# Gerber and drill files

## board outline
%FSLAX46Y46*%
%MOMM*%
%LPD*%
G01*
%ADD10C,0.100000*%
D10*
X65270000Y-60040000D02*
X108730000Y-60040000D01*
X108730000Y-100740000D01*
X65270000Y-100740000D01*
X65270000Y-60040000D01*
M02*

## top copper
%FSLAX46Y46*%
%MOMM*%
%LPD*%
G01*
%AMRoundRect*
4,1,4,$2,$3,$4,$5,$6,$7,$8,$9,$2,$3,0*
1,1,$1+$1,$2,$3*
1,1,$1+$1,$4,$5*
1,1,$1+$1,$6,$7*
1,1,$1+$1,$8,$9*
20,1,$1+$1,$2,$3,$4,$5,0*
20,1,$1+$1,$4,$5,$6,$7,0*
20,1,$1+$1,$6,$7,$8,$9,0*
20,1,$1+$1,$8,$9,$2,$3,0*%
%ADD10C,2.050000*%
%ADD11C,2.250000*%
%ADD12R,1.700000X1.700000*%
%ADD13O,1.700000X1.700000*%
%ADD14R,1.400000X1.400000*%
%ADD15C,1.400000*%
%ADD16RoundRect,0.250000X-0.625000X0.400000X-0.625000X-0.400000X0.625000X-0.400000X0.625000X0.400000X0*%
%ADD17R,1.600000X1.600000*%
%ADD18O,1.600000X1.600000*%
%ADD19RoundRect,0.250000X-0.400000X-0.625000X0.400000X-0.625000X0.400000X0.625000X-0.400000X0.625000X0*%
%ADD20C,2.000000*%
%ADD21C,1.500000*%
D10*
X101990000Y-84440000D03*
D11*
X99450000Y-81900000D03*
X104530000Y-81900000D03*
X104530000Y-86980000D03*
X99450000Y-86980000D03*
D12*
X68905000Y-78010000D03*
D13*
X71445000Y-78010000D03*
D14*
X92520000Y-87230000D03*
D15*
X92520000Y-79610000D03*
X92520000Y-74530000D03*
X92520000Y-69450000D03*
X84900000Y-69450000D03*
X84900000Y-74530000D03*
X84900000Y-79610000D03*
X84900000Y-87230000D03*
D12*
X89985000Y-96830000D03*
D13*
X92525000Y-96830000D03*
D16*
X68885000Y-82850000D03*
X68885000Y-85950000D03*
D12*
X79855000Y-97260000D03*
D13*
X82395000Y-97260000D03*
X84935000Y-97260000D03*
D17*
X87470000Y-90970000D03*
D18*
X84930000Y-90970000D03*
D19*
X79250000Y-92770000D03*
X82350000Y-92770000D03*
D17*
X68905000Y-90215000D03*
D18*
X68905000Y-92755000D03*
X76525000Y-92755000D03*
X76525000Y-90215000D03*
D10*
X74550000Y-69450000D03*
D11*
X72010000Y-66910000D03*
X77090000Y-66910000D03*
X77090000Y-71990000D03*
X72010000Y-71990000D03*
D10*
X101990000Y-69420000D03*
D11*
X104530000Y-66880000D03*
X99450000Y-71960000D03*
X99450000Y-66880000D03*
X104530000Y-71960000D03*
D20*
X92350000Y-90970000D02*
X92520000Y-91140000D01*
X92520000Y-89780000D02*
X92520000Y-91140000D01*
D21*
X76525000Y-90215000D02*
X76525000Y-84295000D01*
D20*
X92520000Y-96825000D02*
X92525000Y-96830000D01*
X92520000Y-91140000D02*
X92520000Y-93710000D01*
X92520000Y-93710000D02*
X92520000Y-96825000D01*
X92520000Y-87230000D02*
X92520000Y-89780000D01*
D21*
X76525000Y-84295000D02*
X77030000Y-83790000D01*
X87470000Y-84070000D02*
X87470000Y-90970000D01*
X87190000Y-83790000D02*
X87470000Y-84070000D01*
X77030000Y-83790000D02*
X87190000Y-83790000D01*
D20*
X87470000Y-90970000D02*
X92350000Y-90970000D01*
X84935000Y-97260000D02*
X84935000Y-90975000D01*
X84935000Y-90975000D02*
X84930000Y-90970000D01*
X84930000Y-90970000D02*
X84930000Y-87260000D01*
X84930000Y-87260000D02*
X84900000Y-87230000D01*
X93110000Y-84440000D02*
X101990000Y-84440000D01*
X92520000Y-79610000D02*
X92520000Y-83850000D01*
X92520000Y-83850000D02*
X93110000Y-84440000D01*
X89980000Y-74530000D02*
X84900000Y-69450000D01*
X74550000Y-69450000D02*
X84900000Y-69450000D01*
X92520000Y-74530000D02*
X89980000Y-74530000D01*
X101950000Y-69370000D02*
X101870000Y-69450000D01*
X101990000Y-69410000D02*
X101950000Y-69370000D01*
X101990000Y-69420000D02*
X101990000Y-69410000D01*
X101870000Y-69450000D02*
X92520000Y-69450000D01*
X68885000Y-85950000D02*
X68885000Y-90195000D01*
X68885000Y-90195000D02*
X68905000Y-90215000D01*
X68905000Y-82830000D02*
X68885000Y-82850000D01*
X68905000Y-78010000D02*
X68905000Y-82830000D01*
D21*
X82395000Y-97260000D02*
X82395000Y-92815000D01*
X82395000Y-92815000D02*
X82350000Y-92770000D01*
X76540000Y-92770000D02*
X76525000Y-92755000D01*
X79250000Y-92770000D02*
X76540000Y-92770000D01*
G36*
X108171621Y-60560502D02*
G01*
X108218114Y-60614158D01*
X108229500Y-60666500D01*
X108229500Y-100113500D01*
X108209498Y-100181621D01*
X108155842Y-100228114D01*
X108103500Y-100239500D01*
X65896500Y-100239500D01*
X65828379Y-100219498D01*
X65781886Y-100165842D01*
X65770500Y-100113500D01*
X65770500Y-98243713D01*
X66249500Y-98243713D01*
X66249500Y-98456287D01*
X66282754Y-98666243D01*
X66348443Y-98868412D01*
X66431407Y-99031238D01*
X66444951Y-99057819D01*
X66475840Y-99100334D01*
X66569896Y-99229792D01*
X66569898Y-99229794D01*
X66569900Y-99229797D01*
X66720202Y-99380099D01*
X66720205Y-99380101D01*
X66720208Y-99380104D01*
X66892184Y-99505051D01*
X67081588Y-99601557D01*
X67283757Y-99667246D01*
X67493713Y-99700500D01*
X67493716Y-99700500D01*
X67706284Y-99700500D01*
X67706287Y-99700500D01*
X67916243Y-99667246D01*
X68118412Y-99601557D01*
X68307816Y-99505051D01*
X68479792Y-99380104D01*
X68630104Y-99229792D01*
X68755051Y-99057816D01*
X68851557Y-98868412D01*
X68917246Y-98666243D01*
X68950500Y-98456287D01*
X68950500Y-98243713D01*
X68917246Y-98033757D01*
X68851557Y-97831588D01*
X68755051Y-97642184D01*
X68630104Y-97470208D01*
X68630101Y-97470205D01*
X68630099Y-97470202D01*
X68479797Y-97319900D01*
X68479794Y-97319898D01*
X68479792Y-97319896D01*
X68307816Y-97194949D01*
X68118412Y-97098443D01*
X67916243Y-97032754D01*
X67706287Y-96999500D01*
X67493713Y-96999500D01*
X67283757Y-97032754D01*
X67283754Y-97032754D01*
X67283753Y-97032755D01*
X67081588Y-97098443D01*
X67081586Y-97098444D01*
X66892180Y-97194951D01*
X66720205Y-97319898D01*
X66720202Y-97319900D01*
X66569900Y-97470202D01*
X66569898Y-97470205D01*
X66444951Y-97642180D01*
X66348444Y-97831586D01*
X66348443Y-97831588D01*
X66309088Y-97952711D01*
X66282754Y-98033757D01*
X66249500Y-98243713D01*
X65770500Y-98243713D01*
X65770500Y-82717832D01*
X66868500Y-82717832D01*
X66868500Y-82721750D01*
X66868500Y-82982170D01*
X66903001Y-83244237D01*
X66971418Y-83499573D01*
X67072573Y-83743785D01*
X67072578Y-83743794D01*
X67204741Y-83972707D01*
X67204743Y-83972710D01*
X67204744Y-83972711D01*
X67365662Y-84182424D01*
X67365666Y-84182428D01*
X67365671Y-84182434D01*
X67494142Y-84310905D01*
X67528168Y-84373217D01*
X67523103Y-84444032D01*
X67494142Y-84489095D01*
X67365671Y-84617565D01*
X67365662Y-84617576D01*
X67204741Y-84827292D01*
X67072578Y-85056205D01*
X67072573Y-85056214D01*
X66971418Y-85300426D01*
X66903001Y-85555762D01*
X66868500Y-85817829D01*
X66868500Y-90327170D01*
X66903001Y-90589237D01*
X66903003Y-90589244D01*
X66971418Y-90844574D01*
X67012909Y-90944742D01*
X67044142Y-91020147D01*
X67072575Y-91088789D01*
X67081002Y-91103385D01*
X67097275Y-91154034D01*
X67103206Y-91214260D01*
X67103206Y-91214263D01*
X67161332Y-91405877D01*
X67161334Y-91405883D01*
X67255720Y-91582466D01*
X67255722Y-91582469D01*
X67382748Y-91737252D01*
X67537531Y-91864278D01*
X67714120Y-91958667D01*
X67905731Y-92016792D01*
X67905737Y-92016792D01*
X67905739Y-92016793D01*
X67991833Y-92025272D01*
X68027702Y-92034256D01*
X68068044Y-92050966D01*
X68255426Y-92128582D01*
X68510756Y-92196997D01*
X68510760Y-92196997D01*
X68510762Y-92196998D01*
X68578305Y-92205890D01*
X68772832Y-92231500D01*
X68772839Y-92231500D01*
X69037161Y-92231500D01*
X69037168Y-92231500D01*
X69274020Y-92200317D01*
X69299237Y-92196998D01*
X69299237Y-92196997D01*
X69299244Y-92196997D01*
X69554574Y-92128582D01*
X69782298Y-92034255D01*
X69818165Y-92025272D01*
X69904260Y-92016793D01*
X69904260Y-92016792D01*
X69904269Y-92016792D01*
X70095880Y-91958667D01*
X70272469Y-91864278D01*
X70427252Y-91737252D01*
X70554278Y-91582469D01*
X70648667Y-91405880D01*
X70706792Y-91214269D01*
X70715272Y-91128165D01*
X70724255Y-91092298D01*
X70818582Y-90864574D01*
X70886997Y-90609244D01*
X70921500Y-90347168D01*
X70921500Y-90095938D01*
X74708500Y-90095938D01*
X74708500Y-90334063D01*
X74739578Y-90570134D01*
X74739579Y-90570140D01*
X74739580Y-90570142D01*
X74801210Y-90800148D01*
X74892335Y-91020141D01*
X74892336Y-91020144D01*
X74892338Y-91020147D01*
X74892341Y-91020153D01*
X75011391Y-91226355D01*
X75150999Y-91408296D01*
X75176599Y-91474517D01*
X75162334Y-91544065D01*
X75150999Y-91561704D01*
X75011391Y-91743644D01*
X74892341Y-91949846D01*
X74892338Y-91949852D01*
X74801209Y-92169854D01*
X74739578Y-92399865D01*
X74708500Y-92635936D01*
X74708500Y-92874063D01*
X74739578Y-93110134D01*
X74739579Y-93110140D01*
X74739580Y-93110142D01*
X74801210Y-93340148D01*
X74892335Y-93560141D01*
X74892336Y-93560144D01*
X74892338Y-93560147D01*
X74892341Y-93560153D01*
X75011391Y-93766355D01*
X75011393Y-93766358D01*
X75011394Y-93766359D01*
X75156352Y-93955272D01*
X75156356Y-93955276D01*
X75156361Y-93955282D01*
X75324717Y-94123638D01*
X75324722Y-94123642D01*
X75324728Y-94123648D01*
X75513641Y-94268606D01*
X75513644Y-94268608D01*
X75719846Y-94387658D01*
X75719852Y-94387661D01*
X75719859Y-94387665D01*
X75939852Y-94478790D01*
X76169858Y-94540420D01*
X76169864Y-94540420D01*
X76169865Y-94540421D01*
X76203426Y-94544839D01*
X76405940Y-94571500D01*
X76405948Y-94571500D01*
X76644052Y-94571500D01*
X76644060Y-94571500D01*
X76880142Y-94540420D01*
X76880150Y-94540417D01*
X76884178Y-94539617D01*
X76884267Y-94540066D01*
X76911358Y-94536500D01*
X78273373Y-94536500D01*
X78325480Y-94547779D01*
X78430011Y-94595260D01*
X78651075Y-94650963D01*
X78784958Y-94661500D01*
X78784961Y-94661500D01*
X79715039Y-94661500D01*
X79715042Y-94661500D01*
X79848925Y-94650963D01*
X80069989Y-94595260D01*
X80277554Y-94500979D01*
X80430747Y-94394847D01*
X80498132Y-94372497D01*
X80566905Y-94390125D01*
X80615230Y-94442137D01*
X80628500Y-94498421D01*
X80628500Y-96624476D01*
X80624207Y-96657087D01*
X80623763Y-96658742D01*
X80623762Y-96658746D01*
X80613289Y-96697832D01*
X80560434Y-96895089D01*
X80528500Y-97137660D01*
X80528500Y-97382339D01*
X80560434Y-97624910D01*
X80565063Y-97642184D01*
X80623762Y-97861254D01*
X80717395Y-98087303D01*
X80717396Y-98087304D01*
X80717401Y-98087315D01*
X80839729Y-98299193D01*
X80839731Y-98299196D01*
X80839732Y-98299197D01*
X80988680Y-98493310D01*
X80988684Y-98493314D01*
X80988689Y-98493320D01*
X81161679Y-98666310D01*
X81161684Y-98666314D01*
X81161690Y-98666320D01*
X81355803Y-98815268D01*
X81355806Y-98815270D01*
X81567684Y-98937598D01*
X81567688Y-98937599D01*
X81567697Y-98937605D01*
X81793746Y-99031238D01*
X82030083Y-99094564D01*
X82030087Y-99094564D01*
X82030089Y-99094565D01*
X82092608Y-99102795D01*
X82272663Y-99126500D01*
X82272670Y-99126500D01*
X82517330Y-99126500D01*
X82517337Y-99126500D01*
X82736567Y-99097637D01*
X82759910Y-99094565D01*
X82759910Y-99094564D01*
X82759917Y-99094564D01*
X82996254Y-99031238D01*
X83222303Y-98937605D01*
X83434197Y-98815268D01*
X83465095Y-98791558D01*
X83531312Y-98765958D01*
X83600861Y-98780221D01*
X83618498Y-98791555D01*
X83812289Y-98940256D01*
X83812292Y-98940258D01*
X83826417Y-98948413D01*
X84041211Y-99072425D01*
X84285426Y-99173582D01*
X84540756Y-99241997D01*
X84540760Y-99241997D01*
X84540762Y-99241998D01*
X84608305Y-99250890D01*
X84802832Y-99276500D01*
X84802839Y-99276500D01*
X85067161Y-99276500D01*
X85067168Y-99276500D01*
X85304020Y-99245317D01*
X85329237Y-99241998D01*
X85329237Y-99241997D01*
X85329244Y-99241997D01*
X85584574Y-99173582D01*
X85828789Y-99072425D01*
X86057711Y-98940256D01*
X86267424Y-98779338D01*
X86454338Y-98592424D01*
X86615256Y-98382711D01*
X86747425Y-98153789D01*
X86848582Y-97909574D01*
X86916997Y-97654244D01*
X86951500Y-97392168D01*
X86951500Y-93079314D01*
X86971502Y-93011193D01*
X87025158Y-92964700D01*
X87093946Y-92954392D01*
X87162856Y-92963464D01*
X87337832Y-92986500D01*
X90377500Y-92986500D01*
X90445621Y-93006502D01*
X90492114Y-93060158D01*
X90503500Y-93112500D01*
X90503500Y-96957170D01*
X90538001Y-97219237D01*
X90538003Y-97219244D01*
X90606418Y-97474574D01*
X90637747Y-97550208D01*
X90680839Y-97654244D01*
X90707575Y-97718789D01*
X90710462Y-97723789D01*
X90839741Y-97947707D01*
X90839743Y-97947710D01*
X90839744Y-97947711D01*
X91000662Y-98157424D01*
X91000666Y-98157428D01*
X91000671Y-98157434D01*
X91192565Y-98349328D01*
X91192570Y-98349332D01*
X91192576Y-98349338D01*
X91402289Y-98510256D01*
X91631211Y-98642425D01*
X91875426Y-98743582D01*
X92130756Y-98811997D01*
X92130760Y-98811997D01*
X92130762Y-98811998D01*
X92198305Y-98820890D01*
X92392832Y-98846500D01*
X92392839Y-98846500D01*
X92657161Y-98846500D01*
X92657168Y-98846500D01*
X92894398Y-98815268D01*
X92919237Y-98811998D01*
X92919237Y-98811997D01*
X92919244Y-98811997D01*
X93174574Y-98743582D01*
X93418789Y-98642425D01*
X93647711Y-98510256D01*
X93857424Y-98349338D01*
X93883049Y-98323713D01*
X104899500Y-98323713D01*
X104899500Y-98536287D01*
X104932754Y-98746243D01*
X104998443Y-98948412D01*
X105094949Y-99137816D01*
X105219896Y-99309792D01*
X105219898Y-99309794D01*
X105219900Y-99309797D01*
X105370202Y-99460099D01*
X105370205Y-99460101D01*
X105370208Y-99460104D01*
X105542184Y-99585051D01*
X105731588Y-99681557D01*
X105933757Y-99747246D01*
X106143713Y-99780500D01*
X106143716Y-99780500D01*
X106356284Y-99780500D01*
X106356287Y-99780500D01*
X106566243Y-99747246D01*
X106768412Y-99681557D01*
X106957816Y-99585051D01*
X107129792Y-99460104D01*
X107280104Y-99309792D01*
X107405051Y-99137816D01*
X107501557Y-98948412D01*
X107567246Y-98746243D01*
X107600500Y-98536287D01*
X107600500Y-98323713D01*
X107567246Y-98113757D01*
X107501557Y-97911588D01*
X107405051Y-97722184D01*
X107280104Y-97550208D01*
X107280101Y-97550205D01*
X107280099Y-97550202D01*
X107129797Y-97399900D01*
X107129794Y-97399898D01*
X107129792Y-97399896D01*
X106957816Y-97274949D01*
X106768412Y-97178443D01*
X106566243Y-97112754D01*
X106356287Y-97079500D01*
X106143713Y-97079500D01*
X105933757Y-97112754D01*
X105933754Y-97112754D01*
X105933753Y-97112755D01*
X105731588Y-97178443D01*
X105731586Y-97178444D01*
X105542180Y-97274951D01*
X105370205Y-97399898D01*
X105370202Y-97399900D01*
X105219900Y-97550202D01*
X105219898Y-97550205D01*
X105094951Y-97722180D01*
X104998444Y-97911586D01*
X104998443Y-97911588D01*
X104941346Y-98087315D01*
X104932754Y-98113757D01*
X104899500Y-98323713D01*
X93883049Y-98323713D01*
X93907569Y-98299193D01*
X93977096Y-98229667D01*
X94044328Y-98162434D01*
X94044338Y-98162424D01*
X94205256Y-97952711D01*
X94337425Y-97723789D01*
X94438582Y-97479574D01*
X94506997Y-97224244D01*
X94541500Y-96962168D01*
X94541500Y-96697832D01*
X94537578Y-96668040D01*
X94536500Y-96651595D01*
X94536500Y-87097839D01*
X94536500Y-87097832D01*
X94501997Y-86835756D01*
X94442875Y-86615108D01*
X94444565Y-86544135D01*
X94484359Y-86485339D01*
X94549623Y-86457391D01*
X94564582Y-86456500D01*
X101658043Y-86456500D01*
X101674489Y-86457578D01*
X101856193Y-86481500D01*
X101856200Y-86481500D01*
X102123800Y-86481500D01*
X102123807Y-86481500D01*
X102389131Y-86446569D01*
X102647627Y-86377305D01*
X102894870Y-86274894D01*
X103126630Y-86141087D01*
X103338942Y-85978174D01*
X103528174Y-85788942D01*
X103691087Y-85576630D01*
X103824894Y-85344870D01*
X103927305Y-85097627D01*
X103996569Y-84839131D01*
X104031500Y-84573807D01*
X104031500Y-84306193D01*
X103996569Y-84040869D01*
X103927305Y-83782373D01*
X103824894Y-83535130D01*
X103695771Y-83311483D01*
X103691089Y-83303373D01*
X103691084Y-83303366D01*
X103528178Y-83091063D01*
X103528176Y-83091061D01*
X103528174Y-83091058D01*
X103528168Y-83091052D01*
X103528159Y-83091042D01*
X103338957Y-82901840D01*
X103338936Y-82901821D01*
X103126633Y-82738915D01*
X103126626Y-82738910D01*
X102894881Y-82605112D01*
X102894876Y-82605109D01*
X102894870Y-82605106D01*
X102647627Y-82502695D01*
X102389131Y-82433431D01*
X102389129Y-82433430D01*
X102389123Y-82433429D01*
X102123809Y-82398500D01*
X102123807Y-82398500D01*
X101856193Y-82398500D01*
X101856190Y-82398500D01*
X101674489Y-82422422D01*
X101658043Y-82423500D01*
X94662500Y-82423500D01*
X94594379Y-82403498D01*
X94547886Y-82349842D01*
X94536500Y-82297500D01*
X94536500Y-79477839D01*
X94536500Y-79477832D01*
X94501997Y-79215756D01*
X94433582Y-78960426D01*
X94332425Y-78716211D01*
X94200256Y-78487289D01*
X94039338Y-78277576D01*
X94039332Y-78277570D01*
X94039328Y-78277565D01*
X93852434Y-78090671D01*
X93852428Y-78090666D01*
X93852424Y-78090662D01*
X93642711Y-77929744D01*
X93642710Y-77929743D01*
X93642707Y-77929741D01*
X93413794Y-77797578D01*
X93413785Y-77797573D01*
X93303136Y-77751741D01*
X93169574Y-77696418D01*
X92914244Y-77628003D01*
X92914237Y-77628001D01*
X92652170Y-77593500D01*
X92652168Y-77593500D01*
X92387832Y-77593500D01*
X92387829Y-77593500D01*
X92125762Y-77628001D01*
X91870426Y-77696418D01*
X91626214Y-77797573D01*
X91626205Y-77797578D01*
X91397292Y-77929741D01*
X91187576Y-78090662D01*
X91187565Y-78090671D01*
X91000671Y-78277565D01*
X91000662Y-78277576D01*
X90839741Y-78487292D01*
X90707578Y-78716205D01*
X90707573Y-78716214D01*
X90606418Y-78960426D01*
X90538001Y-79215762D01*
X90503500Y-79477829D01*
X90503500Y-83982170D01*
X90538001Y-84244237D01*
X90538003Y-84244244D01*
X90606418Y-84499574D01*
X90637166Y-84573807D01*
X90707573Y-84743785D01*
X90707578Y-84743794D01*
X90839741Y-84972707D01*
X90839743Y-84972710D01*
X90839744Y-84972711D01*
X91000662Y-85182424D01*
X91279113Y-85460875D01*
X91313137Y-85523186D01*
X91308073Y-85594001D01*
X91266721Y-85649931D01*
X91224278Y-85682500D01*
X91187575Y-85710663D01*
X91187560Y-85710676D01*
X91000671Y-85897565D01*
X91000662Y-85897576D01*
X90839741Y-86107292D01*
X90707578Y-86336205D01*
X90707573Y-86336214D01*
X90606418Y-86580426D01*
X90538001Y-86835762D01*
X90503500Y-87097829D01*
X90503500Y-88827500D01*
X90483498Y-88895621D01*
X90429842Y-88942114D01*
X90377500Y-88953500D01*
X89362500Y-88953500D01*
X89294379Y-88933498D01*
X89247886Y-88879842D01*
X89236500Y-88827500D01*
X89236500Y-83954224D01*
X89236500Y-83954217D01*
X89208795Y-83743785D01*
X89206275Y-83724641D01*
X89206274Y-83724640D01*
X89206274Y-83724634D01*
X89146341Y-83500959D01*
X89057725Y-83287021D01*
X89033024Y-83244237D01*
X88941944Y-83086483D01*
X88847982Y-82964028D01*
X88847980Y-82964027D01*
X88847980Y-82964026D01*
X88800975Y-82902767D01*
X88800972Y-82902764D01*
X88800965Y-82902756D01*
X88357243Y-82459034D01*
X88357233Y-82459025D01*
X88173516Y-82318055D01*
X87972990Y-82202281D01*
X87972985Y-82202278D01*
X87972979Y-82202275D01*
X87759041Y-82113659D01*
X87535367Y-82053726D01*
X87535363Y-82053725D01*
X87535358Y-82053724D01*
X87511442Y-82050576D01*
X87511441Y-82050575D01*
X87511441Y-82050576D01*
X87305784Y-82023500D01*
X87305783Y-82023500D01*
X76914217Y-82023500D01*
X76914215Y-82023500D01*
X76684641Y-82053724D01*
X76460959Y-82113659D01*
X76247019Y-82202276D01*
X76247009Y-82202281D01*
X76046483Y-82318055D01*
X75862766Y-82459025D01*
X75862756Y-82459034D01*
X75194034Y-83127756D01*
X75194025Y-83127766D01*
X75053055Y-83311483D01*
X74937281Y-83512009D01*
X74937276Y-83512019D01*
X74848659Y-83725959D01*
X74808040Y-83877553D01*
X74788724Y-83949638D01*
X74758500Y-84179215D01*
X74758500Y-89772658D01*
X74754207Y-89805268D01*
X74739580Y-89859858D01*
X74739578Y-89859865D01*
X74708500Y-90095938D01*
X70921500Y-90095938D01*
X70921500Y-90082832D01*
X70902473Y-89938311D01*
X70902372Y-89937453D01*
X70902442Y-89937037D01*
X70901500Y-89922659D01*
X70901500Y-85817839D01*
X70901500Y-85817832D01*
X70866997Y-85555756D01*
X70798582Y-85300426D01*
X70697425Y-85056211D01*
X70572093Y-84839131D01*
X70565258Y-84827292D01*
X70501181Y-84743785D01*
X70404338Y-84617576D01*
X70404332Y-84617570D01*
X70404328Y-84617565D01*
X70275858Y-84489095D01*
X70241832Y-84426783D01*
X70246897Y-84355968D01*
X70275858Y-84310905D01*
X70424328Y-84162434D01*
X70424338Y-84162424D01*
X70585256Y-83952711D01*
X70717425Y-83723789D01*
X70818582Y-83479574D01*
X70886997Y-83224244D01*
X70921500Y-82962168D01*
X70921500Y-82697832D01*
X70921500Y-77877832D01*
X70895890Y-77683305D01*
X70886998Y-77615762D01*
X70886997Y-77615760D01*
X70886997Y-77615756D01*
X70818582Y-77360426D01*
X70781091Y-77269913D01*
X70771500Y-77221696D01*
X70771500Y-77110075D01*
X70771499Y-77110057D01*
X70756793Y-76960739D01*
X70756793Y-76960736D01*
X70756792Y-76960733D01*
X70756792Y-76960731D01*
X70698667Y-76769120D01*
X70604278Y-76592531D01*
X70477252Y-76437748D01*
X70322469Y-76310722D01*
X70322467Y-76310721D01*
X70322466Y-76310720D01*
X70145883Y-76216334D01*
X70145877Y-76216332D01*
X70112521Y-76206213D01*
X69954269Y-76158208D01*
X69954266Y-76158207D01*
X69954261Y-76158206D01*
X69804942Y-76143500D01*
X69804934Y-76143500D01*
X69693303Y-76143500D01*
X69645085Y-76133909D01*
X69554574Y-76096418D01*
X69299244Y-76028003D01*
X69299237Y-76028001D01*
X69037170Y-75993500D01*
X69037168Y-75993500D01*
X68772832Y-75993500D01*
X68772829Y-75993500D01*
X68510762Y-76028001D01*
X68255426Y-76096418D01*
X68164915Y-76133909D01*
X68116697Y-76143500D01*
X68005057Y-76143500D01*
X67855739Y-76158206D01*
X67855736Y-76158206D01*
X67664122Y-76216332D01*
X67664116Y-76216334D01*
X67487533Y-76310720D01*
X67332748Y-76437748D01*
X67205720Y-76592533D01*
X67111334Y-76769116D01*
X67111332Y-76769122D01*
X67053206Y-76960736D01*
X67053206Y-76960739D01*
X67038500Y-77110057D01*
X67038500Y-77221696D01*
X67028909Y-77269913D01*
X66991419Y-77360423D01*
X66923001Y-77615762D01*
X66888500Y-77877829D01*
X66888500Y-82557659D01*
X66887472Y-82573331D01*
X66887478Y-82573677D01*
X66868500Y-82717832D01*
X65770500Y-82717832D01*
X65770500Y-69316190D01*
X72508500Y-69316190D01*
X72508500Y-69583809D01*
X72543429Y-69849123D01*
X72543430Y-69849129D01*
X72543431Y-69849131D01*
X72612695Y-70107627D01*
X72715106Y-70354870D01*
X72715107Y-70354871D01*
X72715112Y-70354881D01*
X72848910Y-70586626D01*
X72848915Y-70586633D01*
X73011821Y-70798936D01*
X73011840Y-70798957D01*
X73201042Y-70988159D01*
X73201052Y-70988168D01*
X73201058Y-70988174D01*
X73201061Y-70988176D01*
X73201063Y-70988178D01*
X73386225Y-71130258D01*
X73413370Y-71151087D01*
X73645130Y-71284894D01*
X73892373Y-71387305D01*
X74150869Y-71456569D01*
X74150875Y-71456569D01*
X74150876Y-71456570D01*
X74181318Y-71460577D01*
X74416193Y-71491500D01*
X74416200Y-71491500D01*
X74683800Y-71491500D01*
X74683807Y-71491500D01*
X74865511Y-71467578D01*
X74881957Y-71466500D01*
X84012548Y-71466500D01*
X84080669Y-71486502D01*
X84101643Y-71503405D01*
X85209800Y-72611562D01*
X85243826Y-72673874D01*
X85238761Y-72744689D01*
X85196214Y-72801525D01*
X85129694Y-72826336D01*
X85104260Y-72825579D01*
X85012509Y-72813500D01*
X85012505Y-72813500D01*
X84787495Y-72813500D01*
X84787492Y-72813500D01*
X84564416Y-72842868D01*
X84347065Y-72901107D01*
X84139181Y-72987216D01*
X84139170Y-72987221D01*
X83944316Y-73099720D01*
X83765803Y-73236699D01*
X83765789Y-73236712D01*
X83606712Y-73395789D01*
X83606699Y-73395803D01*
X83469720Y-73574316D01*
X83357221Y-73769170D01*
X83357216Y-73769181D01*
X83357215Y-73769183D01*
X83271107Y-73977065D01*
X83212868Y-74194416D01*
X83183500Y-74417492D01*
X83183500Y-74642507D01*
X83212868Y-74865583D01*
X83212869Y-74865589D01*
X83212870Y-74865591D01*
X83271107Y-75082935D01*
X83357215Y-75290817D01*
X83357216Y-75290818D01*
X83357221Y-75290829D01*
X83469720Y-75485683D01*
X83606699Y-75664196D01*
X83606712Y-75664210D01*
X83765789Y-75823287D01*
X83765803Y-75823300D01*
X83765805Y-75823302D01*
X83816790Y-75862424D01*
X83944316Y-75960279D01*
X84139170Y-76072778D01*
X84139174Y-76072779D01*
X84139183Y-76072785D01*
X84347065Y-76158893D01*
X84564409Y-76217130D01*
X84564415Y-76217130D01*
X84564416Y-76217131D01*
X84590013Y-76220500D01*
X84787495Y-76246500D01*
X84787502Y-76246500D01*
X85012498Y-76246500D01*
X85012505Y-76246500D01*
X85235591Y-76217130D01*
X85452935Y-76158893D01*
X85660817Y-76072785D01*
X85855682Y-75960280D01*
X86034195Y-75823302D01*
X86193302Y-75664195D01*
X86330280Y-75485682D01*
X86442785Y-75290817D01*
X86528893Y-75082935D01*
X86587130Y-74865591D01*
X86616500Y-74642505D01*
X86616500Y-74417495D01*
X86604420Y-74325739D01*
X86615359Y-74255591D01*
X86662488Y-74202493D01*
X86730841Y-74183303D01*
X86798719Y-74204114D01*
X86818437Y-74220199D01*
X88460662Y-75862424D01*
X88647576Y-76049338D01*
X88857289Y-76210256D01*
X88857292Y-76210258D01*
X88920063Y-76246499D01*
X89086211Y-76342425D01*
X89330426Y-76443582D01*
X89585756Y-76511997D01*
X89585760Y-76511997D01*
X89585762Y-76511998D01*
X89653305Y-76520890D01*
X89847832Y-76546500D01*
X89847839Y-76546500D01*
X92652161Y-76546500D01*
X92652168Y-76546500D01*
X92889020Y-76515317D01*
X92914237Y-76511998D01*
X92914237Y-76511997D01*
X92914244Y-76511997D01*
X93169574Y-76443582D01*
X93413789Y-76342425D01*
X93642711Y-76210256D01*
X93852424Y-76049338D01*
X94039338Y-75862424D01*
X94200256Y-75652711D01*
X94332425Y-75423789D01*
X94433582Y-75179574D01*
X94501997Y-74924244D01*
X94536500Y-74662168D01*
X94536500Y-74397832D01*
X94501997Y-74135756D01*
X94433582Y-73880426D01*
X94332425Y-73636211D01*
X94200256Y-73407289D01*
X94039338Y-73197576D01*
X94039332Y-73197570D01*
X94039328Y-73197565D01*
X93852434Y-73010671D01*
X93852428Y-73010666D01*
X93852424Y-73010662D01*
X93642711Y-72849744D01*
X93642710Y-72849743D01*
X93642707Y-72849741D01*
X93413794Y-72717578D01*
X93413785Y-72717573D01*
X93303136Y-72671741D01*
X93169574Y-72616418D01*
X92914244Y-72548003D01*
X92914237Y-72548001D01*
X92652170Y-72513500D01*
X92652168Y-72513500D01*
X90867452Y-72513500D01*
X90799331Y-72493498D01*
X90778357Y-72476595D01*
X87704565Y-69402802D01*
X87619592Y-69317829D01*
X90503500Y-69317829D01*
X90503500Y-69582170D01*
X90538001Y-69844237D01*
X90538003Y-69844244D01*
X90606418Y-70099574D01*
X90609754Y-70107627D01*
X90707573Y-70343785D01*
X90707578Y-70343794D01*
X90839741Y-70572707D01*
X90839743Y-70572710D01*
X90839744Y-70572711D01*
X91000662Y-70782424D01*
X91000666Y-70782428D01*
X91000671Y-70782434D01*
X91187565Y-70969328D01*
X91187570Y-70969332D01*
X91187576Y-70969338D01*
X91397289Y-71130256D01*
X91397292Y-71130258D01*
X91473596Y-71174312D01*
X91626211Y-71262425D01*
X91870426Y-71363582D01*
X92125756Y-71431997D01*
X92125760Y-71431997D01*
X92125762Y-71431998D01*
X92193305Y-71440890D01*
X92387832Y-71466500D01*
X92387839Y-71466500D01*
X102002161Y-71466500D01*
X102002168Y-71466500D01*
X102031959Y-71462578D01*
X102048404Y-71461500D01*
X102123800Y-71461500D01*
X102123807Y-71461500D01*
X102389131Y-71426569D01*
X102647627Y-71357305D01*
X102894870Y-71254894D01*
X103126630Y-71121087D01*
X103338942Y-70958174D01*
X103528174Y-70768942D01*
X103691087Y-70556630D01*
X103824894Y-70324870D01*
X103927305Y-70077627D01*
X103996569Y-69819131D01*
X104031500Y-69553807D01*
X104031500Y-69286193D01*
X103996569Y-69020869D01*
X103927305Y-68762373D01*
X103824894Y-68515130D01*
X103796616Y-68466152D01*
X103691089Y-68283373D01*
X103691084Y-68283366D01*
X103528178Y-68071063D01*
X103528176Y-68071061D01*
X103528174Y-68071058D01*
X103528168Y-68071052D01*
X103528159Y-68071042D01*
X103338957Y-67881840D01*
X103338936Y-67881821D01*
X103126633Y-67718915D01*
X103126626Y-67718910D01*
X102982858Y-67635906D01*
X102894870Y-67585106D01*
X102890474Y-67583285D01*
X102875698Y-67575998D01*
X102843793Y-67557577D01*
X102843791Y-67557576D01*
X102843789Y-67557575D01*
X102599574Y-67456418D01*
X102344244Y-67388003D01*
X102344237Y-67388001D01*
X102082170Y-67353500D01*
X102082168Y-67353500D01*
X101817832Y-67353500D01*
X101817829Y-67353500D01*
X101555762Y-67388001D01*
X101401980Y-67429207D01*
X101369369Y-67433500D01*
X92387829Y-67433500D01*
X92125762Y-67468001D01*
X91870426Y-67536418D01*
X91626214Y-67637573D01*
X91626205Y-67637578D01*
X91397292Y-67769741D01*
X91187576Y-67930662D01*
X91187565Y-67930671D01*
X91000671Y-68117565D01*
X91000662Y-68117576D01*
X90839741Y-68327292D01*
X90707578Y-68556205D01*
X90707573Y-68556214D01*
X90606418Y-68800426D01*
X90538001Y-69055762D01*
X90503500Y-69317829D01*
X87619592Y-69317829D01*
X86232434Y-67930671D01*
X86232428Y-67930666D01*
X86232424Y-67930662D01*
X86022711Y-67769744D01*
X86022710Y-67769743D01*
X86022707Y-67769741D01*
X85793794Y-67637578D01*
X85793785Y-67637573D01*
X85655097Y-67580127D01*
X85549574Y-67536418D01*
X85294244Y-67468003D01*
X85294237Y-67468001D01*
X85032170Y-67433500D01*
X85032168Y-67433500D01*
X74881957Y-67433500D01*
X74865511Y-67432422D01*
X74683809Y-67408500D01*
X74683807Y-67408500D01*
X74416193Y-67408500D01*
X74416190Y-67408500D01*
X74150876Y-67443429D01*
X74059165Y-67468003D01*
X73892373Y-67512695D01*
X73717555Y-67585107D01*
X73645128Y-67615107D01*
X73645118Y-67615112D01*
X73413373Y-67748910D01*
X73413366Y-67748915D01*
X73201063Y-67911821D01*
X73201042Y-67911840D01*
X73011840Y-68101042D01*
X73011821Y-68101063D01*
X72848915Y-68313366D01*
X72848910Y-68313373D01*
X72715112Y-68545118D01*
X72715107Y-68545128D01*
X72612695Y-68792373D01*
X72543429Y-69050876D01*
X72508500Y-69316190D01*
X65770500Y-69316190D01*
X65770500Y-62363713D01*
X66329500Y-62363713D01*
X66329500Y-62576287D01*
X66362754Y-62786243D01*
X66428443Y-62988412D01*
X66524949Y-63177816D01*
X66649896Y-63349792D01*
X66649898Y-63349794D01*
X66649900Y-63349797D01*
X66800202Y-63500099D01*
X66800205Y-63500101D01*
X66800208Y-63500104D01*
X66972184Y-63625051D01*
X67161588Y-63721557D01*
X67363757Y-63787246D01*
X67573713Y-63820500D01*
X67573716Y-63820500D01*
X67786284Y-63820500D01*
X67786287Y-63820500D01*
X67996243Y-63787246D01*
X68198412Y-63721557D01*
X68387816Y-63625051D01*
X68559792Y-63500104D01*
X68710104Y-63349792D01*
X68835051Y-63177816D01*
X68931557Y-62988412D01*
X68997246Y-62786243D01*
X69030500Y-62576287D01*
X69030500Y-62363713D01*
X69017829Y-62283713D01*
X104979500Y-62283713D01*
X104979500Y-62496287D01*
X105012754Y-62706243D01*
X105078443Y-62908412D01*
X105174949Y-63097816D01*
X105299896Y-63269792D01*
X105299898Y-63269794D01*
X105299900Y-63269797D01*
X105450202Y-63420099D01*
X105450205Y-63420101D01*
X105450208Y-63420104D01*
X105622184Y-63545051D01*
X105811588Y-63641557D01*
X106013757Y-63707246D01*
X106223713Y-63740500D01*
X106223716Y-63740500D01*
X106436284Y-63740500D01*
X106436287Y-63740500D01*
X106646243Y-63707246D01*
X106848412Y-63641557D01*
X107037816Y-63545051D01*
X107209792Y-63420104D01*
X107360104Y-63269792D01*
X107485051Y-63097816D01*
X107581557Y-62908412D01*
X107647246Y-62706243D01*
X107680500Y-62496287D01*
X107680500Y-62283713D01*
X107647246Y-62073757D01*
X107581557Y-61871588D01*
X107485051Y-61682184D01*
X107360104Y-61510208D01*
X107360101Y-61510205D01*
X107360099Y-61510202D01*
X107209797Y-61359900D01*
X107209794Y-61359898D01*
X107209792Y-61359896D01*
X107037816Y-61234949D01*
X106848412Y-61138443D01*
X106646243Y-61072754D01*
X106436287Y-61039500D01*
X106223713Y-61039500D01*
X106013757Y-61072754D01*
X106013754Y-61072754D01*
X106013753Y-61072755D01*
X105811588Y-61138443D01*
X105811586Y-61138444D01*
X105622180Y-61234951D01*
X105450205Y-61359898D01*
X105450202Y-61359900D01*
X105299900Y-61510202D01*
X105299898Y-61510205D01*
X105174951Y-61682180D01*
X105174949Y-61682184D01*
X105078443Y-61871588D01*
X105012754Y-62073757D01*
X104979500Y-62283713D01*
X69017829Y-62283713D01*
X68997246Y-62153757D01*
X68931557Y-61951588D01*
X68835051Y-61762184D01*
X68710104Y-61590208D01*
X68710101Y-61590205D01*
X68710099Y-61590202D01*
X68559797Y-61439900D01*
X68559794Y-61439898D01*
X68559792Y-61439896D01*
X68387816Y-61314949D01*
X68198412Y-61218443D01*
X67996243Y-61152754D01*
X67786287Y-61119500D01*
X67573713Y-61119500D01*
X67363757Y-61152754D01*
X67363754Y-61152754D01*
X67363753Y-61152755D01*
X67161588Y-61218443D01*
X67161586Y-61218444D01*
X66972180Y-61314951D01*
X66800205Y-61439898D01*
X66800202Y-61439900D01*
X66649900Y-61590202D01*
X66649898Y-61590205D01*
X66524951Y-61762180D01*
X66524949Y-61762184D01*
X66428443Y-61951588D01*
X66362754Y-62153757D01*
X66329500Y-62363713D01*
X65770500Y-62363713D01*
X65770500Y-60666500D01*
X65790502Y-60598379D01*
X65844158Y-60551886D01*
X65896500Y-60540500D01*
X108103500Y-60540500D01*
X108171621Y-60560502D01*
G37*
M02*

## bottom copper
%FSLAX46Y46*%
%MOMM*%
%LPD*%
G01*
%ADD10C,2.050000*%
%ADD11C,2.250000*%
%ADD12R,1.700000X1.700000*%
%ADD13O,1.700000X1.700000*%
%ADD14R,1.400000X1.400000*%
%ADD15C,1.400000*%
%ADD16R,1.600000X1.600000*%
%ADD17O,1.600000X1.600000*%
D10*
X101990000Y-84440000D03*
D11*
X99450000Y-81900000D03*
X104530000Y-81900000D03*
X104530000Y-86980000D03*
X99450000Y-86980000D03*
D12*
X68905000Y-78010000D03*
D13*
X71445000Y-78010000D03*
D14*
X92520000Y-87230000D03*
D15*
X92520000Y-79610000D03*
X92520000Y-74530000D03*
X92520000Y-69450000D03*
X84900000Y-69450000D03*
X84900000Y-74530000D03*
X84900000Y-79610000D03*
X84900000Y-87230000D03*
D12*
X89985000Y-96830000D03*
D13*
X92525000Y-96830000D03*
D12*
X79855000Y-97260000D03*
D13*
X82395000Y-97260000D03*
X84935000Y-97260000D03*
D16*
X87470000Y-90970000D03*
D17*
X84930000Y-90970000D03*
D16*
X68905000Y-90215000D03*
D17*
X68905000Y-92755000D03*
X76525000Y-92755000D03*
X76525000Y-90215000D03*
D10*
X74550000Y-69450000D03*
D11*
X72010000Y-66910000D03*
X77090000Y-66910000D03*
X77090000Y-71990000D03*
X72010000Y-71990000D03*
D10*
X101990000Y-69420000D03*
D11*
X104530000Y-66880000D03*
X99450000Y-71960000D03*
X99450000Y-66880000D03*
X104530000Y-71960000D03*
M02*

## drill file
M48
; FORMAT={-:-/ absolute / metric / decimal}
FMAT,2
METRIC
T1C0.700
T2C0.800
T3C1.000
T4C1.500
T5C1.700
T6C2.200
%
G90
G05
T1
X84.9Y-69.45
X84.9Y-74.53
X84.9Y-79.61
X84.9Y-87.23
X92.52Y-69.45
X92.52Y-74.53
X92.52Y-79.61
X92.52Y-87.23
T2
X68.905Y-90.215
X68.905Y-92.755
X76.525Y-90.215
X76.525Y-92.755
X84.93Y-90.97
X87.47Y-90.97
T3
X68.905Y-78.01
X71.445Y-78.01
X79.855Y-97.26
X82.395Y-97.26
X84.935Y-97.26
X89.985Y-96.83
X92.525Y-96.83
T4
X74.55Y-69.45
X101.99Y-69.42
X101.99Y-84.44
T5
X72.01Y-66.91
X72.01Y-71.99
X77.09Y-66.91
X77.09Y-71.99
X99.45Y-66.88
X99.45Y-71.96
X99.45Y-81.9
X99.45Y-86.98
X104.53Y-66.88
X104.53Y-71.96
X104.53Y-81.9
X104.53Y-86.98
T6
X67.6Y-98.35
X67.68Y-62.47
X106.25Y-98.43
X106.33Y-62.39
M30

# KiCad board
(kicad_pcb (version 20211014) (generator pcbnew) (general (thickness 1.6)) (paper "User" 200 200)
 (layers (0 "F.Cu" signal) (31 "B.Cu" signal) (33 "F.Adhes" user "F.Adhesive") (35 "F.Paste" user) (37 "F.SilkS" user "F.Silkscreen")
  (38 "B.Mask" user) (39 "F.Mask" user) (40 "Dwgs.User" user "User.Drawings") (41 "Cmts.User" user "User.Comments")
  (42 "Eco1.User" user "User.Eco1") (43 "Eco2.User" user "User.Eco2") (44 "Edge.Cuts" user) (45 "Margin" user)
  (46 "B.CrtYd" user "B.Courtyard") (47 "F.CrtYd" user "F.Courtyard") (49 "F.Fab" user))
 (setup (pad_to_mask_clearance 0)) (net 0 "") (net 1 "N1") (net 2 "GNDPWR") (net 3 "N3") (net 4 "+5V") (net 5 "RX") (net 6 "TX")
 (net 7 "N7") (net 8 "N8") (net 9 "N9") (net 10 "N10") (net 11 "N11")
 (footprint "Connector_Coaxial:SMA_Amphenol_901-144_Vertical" (layer "F.Cu") (at 101.99 84.44)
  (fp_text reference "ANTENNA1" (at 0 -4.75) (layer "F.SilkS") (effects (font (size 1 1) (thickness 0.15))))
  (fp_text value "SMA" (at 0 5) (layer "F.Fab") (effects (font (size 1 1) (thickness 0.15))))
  (pad "1" thru_hole circle (at 0 0) (size 2.05 2.05) (drill 1.5) (layers *.Cu *.Mask) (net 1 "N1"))
  (pad "2" thru_hole circle (at -2.54 -2.54) (size 2.25 2.25) (drill 1.7) (layers *.Cu *.Mask) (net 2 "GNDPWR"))
  (pad "2" thru_hole circle (at 2.54 -2.54) (size 2.25 2.25) (drill 1.7) (layers *.Cu *.Mask) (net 2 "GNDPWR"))
  (pad "2" thru_hole circle (at 2.54 2.54) (size 2.25 2.25) (drill 1.7) (layers *.Cu *.Mask) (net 2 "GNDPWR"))
  (pad "2" thru_hole circle (at -2.54 2.54) (size 2.25 2.25) (drill 1.7) (layers *.Cu *.Mask) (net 2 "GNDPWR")))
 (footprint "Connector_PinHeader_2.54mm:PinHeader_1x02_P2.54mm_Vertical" (layer "F.Cu") (at 68.905 78.01 90)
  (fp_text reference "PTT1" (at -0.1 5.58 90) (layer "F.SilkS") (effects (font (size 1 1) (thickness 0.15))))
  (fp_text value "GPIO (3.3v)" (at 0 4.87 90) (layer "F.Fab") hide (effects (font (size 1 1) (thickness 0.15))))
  (pad "1" thru_hole rect (at 0 0 90) (size 1.7 1.7) (drill 1) (layers *.Cu *.Mask) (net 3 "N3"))
  (pad "2" thru_hole oval (at 0 2.54 90) (size 1.7 1.7) (drill 1) (layers *.Cu *.Mask) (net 2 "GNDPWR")))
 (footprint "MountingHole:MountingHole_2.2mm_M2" (layer "F.Cu") (at 106.33 62.39)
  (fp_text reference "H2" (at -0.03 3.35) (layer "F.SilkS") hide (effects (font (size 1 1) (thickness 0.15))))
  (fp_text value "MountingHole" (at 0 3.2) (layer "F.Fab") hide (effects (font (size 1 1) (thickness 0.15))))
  (pad "" np_thru_hole circle (at 0 0) (size 2.2 2.2) (drill 2.2) (layers *.Cu *.Mask)))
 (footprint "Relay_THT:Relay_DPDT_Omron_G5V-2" (layer "F.Cu") (at 92.52 87.23 180)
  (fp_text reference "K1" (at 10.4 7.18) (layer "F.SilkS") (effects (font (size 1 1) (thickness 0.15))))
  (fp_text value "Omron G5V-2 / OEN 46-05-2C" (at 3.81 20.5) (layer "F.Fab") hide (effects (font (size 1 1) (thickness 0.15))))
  (pad "1" thru_hole rect (at 0 0 180) (size 1.4 1.4) (drill 0.7) (layers *.Cu *.Mask) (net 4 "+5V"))
  (pad "4" thru_hole circle (at 0 7.62 180) (size 1.4 1.4) (drill 0.7) (layers *.Cu *.Mask) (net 1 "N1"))
  (pad "6" thru_hole circle (at 0 12.7 180) (size 1.4 1.4) (drill 0.7) (layers *.Cu *.Mask) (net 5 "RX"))
  (pad "8" thru_hole circle (at 0 17.78 180) (size 1.4 1.4) (drill 0.7) (layers *.Cu *.Mask) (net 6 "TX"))
  (pad "9" thru_hole circle (at 7.62 17.78 180) (size 1.4 1.4) (drill 0.7) (layers *.Cu *.Mask) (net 5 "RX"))
  (pad "11" thru_hole circle (at 7.62 12.7 180) (size 1.4 1.4) (drill 0.7) (layers *.Cu *.Mask) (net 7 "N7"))
  (pad "13" thru_hole circle (at 7.62 7.62 180) (size 1.4 1.4) (drill 0.7) (layers *.Cu *.Mask) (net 2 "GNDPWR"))
  (pad "16" thru_hole circle (at 7.62 0 180) (size 1.4 1.4) (drill 0.7) (layers *.Cu *.Mask) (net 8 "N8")))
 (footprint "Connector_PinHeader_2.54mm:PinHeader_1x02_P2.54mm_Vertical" (layer "F.Cu") (at 89.985 96.83 90)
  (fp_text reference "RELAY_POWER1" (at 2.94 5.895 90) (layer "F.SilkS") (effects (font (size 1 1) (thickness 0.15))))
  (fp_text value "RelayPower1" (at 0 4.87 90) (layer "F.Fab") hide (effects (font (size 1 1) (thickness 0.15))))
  (pad "1" thru_hole rect (at 0 0 90) (size 1.7 1.7) (drill 1) (layers *.Cu *.Mask) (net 2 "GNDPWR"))
  (pad "2" thru_hole oval (at 0 2.54 90) (size 1.7 1.7) (drill 1) (layers *.Cu *.Mask) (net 4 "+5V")))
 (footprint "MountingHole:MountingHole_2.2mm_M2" (layer "F.Cu") (at 67.68 62.47)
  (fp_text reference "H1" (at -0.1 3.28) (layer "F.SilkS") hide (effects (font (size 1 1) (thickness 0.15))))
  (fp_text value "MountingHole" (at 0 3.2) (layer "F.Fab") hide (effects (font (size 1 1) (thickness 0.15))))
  (pad "" np_thru_hole circle (at 0 0) (size 2.2 2.2) (drill 2.2) (layers *.Cu *.Mask)))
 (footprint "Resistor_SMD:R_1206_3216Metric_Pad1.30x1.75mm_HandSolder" (layer "F.Cu") (at 68.885 84.4 -90)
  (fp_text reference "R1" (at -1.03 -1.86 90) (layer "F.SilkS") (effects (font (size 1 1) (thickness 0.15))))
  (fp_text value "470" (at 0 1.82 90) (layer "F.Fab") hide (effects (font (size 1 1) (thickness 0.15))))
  (pad "1" smd roundrect (at -1.55 0 270) (size 1.3 1.75) (layers "F.Cu" "F.Paste" "F.Mask") (roundrect_rratio 0.192308) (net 3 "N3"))
  (pad "2" smd roundrect (at 1.55 0 270) (size 1.3 1.75) (layers "F.Cu" "F.Paste" "F.Mask") (roundrect_rratio 0.192308) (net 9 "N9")))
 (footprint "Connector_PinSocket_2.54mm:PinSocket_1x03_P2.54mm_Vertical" (layer "F.Cu") (at 79.855 97.26 90)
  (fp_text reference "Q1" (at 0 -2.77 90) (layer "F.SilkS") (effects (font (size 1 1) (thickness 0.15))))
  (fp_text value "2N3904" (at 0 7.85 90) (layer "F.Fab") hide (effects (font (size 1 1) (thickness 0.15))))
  (pad "1" thru_hole rect (at 0 0 90) (size 1.7 1.7) (drill 1) (layers *.Cu *.Mask) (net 2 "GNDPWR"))
  (pad "2" thru_hole oval (at 0 2.54 90) (size 1.7 1.7) (drill 1) (layers *.Cu *.Mask) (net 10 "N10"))
  (pad "3" thru_hole oval (at 0 5.08 90) (size 1.7 1.7) (drill 1) (layers *.Cu *.Mask) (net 8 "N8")))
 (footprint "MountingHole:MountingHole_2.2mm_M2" (layer "F.Cu") (at 106.25 98.43)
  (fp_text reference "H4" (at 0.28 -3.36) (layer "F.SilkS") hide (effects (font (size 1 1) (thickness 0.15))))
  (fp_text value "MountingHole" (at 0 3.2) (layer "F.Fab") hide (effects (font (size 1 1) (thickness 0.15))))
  (pad "" np_thru_hole circle (at 0 0) (size 2.2 2.2) (drill 2.2) (layers *.Cu *.Mask)))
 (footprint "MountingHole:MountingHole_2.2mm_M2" (layer "F.Cu") (at 67.6 98.35)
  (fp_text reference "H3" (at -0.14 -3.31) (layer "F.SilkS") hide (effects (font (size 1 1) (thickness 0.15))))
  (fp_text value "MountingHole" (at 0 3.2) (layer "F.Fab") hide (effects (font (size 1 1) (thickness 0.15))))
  (pad "" np_thru_hole circle (at 0 0) (size 2.2 2.2) (drill 2.2) (layers *.Cu *.Mask)))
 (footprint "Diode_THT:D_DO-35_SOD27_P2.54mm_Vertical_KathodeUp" (layer "F.Cu") (at 87.47 90.97 180)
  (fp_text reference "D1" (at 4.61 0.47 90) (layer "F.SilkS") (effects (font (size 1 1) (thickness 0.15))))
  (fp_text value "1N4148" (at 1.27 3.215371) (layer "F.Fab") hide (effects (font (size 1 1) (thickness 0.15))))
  (pad "1" thru_hole rect (at 0 0 180) (size 1.6 1.6) (drill 0.8) (layers *.Cu *.Mask) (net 4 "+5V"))
  (pad "2" thru_hole oval (at 2.54 0 180) (size 1.6 1.6) (drill 0.8) (layers *.Cu *.Mask) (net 8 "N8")))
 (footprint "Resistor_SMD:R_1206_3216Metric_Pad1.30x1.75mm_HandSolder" (layer "F.Cu") (at 80.8 92.77)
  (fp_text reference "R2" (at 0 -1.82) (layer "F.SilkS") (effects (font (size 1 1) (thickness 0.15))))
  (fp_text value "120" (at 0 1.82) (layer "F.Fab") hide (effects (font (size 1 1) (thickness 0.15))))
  (pad "1" smd roundrect (at -1.55 0) (size 1.3 1.75) (layers "F.Cu" "F.Paste" "F.Mask") (roundrect_rratio 0.192308) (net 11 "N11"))
  (pad "2" smd roundrect (at 1.55 0) (size 1.3 1.75) (layers "F.Cu" "F.Paste" "F.Mask") (roundrect_rratio 0.192308) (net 10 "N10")))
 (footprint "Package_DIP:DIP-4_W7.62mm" (layer "F.Cu") (at 68.905 90.215)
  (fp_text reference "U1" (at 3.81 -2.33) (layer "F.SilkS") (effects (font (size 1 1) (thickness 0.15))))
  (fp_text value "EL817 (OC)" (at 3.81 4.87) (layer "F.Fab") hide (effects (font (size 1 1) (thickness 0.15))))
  (pad "1" thru_hole rect (at 0 0) (size 1.6 1.6) (drill 0.8) (layers *.Cu *.Mask) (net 9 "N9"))
  (pad "2" thru_hole oval (at 0 2.54) (size 1.6 1.6) (drill 0.8) (layers *.Cu *.Mask) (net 2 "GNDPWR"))
  (pad "3" thru_hole oval (at 7.62 2.54) (size 1.6 1.6) (drill 0.8) (layers *.Cu *.Mask) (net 11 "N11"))
  (pad "4" thru_hole oval (at 7.62 0) (size 1.6 1.6) (drill 0.8) (layers *.Cu *.Mask) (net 4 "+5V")))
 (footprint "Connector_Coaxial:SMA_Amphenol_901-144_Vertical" (layer "F.Cu") (at 74.55 69.45)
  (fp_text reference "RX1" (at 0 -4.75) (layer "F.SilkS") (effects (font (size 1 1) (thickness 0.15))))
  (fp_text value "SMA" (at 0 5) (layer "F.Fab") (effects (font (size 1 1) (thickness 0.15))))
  (pad "1" thru_hole circle (at 0 0) (size 2.05 2.05) (drill 1.5) (layers *.Cu *.Mask) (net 5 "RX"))
  (pad "2" thru_hole circle (at -2.54 -2.54) (size 2.25 2.25) (drill 1.7) (layers *.Cu *.Mask) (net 2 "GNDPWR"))
  (pad "2" thru_hole circle (at 2.54 -2.54) (size 2.25 2.25) (drill 1.7) (layers *.Cu *.Mask) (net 2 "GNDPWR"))
  (pad "2" thru_hole circle (at 2.54 2.54) (size 2.25 2.25) (drill 1.7) (layers *.Cu *.Mask) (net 2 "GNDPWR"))
  (pad "2" thru_hole circle (at -2.54 2.54) (size 2.25 2.25) (drill 1.7) (layers *.Cu *.Mask) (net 2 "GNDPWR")))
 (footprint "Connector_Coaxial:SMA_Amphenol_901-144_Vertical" (layer "F.Cu") (at 101.99 69.42)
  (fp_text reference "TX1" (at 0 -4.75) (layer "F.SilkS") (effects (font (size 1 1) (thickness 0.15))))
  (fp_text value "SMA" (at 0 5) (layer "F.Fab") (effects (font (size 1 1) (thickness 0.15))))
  (pad "1" thru_hole circle (at 0 0) (size 2.05 2.05) (drill 1.5) (layers *.Cu *.Mask) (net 6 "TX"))
  (pad "2" thru_hole circle (at 2.54 -2.54) (size 2.25 2.25) (drill 1.7) (layers *.Cu *.Mask) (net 2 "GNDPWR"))
  (pad "2" thru_hole circle (at -2.54 2.54) (size 2.25 2.25) (drill 1.7) (layers *.Cu *.Mask) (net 2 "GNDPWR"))
  (pad "2" thru_hole circle (at -2.54 -2.54) (size 2.25 2.25) (drill 1.7) (layers *.Cu *.Mask) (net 2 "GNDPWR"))
  (pad "2" thru_hole circle (at 2.54 2.54) (size 2.25 2.25) (drill 1.7) (layers *.Cu *.Mask) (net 2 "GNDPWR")))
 (gr_rect (start 65.27 60.04) (end 108.73 100.74) (layer "Edge.Cuts") (width 0.1) (fill none))
 (segment (start 92.35 90.97) (end 92.52 91.14) (width 2) (layer "F.Cu") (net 4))
 (segment (start 92.52 89.78) (end 92.52 91.14) (width 2) (layer "F.Cu") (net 4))
 (segment (start 76.525 90.215) (end 76.525 84.295) (width 1.5) (layer "F.Cu") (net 4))
 (segment (start 92.52 96.825) (end 92.525 96.83) (width 2) (layer "F.Cu") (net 4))
 (segment (start 92.52 91.14) (end 92.52 93.71) (width 2) (layer "F.Cu") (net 4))
 (segment (start 92.52 93.71) (end 92.52 96.825) (width 2) (layer "F.Cu") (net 4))
 (segment (start 92.52 87.23) (end 92.52 89.78) (width 2) (layer "F.Cu") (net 4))
 (segment (start 76.525 84.295) (end 77.03 83.79) (width 1.5) (layer "F.Cu") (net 4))
 (segment (start 87.47 84.07) (end 87.47 90.97) (width 1.5) (layer "F.Cu") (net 4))
 (segment (start 87.19 83.79) (end 87.47 84.07) (width 1.5) (layer "F.Cu") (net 4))
 (segment (start 77.03 83.79) (end 87.19 83.79) (width 1.5) (layer "F.Cu") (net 4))
 (segment (start 87.47 90.97) (end 92.35 90.97) (width 2) (layer "F.Cu") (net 4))
 (segment (start 84.935 97.26) (end 84.935 90.975) (width 2) (layer "F.Cu") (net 8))
 (segment (start 84.935 90.975) (end 84.93 90.97) (width 2) (layer "F.Cu") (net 8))
 (segment (start 84.93 90.97) (end 84.93 87.26) (width 2) (layer "F.Cu") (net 8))
 (segment (start 84.93 87.26) (end 84.9 87.23) (width 2) (layer "F.Cu") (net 8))
 (segment (start 93.11 84.44) (end 101.99 84.44) (width 2) (layer "F.Cu") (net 1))
 (segment (start 92.52 79.61) (end 92.52 83.85) (width 2) (layer "F.Cu") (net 1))
 (segment (start 92.52 83.85) (end 93.11 84.44) (width 2) (layer "F.Cu") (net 1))
 (segment (start 89.98 74.53) (end 84.9 69.45) (width 2) (layer "F.Cu") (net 5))
 (segment (start 74.55 69.45) (end 84.9 69.45) (width 2) (layer "F.Cu") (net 5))
 (segment (start 92.52 74.53) (end 89.98 74.53) (width 2) (layer "F.Cu") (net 5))
 (segment (start 101.95 69.37) (end 101.87 69.45) (width 2) (layer "F.Cu") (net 6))
 (segment (start 101.99 69.41) (end 101.95 69.37) (width 2) (layer "F.Cu") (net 6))
 (segment (start 101.99 69.42) (end 101.99 69.41) (width 2) (layer "F.Cu") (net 6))
 (segment (start 101.87 69.45) (end 92.52 69.45) (width 2) (layer "F.Cu") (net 6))
 (segment (start 68.885 85.95) (end 68.885 90.195) (width 2) (layer "F.Cu") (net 9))
 (segment (start 68.885 90.195) (end 68.905 90.215) (width 2) (layer "F.Cu") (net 9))
 (segment (start 68.905 82.83) (end 68.885 82.85) (width 2) (layer "F.Cu") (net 3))
 (segment (start 68.905 78.01) (end 68.905 82.83) (width 2) (layer "F.Cu") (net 3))
 (segment (start 82.395 97.26) (end 82.395 92.815) (width 1.5) (layer "F.Cu") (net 10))
 (segment (start 82.395 92.815) (end 82.35 92.77) (width 1.5) (layer "F.Cu") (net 10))
 (segment (start 76.54 92.77) (end 76.525 92.755) (width 1.5) (layer "F.Cu") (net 11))
 (segment (start 79.25 92.77) (end 76.54 92.77) (width 1.5) (layer "F.Cu") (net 11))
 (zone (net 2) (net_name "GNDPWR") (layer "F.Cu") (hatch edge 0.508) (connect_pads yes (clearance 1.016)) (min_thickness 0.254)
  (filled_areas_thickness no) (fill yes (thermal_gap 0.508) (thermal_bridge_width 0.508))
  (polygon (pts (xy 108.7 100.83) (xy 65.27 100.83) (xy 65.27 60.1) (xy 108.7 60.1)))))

